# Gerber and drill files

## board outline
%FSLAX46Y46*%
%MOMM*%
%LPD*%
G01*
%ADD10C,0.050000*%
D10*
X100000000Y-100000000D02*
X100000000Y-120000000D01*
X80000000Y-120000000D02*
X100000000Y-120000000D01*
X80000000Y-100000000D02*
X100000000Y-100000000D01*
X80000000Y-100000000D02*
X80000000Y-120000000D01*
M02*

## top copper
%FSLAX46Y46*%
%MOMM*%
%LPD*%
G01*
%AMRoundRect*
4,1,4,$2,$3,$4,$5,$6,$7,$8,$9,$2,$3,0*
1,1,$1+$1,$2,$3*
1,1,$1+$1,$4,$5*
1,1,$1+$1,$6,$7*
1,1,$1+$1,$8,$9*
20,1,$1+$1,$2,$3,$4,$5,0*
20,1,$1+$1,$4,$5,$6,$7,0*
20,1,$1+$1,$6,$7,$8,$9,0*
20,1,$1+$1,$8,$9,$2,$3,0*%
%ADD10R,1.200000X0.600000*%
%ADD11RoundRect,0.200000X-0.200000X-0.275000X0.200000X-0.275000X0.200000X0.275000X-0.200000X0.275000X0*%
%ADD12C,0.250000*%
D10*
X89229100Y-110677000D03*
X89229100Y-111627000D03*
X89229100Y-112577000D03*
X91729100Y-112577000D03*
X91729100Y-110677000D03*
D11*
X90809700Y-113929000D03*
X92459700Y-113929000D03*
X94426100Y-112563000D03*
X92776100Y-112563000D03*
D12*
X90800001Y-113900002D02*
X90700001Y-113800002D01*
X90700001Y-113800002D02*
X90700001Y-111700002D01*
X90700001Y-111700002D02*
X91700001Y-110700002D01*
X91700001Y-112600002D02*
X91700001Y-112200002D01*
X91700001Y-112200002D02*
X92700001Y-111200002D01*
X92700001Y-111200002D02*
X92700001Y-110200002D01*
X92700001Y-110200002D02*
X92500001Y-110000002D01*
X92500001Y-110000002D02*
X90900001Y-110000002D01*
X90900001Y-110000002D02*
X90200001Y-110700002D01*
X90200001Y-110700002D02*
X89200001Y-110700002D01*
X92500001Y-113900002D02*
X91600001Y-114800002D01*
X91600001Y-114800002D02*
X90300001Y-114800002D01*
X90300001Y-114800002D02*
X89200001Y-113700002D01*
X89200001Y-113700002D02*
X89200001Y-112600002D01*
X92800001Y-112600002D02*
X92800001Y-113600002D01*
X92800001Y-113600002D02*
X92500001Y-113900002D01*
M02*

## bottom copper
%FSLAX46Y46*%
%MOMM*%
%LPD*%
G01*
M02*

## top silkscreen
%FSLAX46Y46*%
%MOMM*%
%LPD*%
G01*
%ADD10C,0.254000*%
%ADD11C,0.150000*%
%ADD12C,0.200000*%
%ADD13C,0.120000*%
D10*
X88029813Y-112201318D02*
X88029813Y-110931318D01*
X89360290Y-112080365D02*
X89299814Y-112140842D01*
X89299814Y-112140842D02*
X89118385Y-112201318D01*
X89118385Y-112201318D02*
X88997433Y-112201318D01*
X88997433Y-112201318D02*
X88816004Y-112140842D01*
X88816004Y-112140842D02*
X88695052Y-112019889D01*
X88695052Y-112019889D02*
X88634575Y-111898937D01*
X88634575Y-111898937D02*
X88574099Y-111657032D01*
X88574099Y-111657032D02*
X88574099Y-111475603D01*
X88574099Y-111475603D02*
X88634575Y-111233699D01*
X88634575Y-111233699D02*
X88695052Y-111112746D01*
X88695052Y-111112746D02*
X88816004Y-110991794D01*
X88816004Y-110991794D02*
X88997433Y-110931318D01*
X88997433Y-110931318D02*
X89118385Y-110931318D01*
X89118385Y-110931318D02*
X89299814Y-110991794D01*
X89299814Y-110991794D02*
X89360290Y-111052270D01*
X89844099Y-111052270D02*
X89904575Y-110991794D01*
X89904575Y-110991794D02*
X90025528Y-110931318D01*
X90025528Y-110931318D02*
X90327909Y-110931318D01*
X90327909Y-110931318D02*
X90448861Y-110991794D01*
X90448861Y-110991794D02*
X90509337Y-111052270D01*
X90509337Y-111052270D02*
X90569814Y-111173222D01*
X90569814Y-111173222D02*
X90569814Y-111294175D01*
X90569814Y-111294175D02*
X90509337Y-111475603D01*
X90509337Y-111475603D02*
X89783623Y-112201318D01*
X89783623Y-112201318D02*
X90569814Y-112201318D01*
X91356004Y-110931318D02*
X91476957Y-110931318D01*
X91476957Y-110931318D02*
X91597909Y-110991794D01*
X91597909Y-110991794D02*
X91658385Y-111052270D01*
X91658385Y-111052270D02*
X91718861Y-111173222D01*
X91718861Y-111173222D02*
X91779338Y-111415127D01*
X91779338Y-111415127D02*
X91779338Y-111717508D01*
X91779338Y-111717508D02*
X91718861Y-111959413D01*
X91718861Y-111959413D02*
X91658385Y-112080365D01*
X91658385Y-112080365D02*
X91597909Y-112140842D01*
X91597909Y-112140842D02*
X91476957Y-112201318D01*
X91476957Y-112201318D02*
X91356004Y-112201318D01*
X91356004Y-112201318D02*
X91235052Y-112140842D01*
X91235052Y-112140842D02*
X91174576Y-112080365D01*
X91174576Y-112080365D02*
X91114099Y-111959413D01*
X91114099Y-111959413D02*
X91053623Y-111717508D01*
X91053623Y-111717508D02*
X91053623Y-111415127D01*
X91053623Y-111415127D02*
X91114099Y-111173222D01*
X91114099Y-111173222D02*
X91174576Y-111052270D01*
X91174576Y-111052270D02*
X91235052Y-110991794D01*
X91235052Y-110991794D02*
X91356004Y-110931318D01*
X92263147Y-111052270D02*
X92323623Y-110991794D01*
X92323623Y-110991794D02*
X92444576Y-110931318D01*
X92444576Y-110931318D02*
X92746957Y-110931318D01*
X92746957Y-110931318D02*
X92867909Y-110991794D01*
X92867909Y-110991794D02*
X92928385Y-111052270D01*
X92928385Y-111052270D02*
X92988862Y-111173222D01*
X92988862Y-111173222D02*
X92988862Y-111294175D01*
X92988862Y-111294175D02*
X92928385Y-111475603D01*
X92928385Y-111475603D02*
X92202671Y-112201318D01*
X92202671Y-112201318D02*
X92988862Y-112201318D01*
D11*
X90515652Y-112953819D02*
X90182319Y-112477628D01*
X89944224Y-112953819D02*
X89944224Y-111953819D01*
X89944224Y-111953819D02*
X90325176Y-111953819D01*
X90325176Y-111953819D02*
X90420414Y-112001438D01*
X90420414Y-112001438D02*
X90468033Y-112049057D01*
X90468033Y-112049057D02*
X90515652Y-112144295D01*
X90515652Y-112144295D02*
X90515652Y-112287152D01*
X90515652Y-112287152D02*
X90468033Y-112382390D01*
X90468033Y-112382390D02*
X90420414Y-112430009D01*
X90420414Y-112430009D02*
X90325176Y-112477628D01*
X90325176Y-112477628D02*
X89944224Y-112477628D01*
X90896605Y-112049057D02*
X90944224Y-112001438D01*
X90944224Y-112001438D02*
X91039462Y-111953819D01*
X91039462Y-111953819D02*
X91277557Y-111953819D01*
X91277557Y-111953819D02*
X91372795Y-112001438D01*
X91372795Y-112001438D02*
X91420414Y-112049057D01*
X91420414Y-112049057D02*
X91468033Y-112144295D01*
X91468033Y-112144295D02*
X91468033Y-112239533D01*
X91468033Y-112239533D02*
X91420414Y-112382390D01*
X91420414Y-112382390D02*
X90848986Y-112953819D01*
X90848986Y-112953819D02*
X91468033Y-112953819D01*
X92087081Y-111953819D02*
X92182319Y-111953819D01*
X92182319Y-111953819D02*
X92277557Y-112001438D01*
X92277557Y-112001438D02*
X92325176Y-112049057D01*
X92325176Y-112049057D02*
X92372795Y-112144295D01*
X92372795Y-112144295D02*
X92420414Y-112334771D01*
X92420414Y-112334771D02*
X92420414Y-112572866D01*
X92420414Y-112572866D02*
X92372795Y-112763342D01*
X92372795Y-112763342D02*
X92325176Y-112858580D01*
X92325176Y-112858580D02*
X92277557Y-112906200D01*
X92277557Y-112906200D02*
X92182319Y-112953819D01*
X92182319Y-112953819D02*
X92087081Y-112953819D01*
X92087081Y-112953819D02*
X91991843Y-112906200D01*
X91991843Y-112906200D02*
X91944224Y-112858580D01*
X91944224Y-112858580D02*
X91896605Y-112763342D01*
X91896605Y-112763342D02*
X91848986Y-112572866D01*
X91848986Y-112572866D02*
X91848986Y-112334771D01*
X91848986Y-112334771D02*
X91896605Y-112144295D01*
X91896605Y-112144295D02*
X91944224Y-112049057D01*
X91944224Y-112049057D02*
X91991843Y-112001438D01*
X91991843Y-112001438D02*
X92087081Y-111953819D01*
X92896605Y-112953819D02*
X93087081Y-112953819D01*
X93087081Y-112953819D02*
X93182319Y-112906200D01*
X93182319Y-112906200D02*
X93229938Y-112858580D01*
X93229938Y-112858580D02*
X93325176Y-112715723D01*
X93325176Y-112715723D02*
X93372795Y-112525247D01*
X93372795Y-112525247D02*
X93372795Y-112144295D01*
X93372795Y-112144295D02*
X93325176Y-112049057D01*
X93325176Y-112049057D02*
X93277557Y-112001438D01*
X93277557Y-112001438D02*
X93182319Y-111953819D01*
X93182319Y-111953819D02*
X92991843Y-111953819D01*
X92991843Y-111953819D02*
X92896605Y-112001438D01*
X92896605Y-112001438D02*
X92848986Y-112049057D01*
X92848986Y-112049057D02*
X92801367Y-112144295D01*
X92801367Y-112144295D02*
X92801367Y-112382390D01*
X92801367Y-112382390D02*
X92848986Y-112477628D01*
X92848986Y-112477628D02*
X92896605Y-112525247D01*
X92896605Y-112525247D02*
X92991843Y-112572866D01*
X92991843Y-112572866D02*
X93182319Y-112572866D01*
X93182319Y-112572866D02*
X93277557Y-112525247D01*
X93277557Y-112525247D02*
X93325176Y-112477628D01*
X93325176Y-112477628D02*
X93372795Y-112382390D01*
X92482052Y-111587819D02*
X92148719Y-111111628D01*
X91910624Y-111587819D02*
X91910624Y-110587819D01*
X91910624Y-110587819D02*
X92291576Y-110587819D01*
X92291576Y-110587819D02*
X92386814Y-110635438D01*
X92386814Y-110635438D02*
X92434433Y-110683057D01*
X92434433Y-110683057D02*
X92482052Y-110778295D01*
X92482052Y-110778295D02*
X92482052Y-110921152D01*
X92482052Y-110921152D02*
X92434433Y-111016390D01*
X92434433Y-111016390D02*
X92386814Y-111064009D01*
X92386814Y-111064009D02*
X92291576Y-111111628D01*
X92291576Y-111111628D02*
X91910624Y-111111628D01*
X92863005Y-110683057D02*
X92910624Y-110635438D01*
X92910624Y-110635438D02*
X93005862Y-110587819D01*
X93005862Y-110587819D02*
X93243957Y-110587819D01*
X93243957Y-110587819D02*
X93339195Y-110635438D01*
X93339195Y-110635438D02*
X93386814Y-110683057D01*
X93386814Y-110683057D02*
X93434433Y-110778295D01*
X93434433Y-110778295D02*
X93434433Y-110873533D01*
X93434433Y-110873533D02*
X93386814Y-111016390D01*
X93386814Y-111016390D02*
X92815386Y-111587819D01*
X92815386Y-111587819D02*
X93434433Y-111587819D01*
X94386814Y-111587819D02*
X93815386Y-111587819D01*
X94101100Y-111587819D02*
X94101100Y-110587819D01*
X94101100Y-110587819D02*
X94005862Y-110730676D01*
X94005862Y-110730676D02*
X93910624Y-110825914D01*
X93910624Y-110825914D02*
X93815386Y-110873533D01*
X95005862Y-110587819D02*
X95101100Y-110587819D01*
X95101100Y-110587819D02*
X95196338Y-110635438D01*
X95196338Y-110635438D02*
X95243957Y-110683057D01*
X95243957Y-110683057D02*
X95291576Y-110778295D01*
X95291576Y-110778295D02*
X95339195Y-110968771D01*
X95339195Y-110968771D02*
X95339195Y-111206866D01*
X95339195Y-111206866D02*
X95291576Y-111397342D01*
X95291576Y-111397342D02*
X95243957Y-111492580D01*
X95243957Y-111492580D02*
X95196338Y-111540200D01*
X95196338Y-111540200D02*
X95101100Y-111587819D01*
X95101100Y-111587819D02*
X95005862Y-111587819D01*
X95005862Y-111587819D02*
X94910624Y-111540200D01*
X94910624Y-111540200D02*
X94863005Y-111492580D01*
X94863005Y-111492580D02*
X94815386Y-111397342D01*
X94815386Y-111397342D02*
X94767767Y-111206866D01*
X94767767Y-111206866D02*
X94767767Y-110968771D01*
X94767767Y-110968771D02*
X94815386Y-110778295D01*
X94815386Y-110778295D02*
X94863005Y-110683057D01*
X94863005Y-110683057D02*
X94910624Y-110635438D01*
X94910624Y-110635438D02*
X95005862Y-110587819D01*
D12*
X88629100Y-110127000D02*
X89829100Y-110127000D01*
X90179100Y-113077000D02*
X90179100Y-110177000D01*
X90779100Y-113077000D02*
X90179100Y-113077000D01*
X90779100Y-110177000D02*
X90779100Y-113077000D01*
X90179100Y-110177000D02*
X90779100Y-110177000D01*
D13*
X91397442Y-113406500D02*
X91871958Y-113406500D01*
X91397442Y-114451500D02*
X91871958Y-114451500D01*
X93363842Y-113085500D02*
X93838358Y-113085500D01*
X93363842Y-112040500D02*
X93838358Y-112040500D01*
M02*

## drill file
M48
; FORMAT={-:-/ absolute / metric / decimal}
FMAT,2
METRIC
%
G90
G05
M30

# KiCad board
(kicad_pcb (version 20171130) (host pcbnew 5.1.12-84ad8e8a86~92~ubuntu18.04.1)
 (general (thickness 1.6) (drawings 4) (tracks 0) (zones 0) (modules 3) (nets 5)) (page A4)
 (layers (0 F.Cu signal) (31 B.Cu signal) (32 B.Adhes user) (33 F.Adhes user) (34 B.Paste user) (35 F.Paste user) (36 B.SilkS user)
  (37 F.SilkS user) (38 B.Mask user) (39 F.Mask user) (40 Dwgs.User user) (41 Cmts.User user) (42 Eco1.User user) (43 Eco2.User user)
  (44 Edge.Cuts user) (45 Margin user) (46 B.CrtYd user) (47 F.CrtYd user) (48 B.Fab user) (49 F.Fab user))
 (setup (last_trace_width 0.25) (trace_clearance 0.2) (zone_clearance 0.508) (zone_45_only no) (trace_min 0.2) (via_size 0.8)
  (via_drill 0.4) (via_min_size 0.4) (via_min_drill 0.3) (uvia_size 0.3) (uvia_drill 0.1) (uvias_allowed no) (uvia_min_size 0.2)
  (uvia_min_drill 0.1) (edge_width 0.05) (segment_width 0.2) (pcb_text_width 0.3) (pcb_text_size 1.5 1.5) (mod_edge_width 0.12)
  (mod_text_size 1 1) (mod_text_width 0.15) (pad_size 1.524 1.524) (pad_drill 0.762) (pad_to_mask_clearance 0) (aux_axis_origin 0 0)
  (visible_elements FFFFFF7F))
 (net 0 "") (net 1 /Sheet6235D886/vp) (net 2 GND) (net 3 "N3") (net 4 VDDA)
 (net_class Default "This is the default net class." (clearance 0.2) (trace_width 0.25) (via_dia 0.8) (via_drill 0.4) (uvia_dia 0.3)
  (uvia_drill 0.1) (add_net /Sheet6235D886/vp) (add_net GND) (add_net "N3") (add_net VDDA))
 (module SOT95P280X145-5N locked (layer F.Cu) (at 90.479100 111.627000)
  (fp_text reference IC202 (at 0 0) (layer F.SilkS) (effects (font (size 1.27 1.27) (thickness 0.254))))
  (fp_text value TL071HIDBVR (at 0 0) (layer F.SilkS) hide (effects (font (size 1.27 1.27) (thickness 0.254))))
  (fp_line (start -1.85 -1.5) (end -0.65 -1.5) (layer F.SilkS) (width 0.2))
  (fp_line (start -0.3 1.45) (end -0.3 -1.45) (layer F.SilkS) (width 0.2))
  (fp_line (start 0.3 1.45) (end -0.3 1.45) (layer F.SilkS) (width 0.2))
  (fp_line (start 0.3 -1.45) (end 0.3 1.45) (layer F.SilkS) (width 0.2))
  (fp_line (start -0.3 -1.45) (end 0.3 -1.45) (layer F.SilkS) (width 0.2))
  (pad 1 smd rect (at -1.25 -0.95 90.000000) (size 0.6 1.2) (layers F.Cu F.Mask F.Paste) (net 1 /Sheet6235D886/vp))
  (pad 2 smd rect (at -1.25 0 90.000000) (size 0.6 1.2) (layers F.Cu F.Mask F.Paste) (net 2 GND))
  (pad 3 smd rect (at -1.25 0.95 90.000000) (size 0.6 1.2) (layers F.Cu F.Mask F.Paste) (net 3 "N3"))
  (pad 4 smd rect (at 1.25 0.95 90.000000) (size 0.6 1.2) (layers F.Cu F.Mask F.Paste) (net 1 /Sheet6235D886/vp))
  (pad 5 smd rect (at 1.25 -0.95 90.000000) (size 0.6 1.2) (layers F.Cu F.Mask F.Paste) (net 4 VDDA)))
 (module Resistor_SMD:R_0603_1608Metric (layer F.Cu) (at 91.634700 113.929000)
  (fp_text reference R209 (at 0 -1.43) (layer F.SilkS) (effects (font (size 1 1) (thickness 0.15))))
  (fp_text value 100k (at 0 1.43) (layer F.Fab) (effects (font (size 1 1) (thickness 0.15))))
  (fp_line (start -0.237258 -0.5225) (end 0.237258 -0.5225) (layer F.SilkS) (width 0.12))
  (fp_line (start -0.237258 0.5225) (end 0.237258 0.5225) (layer F.SilkS) (width 0.12))
  (pad 1 smd roundrect (at -0.825 0) (size 0.8 0.95) (layers F.Cu F.Mask F.Paste) (roundrect_rratio 0.25) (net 4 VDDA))
  (pad 2 smd roundrect (at 0.825 0) (size 0.8 0.95) (layers F.Cu F.Mask F.Paste) (roundrect_rratio 0.25) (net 3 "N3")))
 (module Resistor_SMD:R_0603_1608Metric (layer F.Cu) (at 93.601100 112.563000)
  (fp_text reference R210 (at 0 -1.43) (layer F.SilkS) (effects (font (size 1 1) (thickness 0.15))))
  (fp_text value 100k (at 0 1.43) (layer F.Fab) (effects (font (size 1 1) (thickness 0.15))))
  (fp_line (start -0.237258 0.5225) (end 0.237258 0.5225) (layer F.SilkS) (width 0.12))
  (fp_line (start -0.237258 -0.5225) (end 0.237258 -0.5225) (layer F.SilkS) (width 0.12))
  (pad 2 smd roundrect (at 0.825 0) (size 0.8 0.95) (layers F.Cu F.Mask F.Paste) (roundrect_rratio 0.25) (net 2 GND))
  (pad 1 smd roundrect (at -0.825 0) (size 0.8 0.95) (layers F.Cu F.Mask F.Paste) (roundrect_rratio 0.25) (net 3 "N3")))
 (gr_line (start 100 100) (end 100 120) (layer Edge.Cuts) (width 0.05))
 (gr_line (start 80 120) (end 100 120) (layer Edge.Cuts) (width 0.05))
 (gr_line (start 80 100) (end 100 100) (layer Edge.Cuts) (width 0.05))
 (gr_line (start 80 100) (end 80 120) (layer Edge.Cuts) (width 0.05))
 (segment (start 90.800001 113.900002) (end 90.700001 113.800002) (width 0.250000) (layer F.Cu) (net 4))
 (segment (start 90.700001 113.800002) (end 90.700001 111.700002) (width 0.250000) (layer F.Cu) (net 4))
 (segment (start 90.700001 111.700002) (end 91.700001 110.700002) (width 0.250000) (layer F.Cu) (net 4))
 (segment (start 91.700001 112.600002) (end 91.700001 112.200002) (width 0.250000) (layer F.Cu) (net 1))
 (segment (start 91.700001 112.200002) (end 92.700001 111.200002) (width 0.250000) (layer F.Cu) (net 1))
 (segment (start 92.700001 111.200002) (end 92.700001 110.200002) (width 0.250000) (layer F.Cu) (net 1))
 (segment (start 92.700001 110.200002) (end 92.500001 110.000002) (width 0.250000) (layer F.Cu) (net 1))
 (segment (start 92.500001 110.000002) (end 90.900001 110.000002) (width 0.250000) (layer F.Cu) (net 1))
 (segment (start 90.900001 110.000002) (end 90.200001 110.700002) (width 0.250000) (layer F.Cu) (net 1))
 (segment (start 90.200001 110.700002) (end 89.200001 110.700002) (width 0.250000) (layer F.Cu) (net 1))
 (segment (start 92.500001 113.900002) (end 91.600001 114.800002) (width 0.250000) (layer F.Cu) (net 3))
 (segment (start 91.600001 114.800002) (end 90.300001 114.800002) (width 0.250000) (layer F.Cu) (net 3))
 (segment (start 90.300001 114.800002) (end 89.200001 113.700002) (width 0.250000) (layer F.Cu) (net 3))
 (segment (start 89.200001 113.700002) (end 89.200001 112.600002) (width 0.250000) (layer F.Cu) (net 3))
 (segment (start 92.800001 112.600002) (end 92.800001 113.600002) (width 0.250000) (layer F.Cu) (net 3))
 (segment (start 92.800001 113.600002) (end 92.500001 113.900002) (width 0.250000) (layer F.Cu) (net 3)))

